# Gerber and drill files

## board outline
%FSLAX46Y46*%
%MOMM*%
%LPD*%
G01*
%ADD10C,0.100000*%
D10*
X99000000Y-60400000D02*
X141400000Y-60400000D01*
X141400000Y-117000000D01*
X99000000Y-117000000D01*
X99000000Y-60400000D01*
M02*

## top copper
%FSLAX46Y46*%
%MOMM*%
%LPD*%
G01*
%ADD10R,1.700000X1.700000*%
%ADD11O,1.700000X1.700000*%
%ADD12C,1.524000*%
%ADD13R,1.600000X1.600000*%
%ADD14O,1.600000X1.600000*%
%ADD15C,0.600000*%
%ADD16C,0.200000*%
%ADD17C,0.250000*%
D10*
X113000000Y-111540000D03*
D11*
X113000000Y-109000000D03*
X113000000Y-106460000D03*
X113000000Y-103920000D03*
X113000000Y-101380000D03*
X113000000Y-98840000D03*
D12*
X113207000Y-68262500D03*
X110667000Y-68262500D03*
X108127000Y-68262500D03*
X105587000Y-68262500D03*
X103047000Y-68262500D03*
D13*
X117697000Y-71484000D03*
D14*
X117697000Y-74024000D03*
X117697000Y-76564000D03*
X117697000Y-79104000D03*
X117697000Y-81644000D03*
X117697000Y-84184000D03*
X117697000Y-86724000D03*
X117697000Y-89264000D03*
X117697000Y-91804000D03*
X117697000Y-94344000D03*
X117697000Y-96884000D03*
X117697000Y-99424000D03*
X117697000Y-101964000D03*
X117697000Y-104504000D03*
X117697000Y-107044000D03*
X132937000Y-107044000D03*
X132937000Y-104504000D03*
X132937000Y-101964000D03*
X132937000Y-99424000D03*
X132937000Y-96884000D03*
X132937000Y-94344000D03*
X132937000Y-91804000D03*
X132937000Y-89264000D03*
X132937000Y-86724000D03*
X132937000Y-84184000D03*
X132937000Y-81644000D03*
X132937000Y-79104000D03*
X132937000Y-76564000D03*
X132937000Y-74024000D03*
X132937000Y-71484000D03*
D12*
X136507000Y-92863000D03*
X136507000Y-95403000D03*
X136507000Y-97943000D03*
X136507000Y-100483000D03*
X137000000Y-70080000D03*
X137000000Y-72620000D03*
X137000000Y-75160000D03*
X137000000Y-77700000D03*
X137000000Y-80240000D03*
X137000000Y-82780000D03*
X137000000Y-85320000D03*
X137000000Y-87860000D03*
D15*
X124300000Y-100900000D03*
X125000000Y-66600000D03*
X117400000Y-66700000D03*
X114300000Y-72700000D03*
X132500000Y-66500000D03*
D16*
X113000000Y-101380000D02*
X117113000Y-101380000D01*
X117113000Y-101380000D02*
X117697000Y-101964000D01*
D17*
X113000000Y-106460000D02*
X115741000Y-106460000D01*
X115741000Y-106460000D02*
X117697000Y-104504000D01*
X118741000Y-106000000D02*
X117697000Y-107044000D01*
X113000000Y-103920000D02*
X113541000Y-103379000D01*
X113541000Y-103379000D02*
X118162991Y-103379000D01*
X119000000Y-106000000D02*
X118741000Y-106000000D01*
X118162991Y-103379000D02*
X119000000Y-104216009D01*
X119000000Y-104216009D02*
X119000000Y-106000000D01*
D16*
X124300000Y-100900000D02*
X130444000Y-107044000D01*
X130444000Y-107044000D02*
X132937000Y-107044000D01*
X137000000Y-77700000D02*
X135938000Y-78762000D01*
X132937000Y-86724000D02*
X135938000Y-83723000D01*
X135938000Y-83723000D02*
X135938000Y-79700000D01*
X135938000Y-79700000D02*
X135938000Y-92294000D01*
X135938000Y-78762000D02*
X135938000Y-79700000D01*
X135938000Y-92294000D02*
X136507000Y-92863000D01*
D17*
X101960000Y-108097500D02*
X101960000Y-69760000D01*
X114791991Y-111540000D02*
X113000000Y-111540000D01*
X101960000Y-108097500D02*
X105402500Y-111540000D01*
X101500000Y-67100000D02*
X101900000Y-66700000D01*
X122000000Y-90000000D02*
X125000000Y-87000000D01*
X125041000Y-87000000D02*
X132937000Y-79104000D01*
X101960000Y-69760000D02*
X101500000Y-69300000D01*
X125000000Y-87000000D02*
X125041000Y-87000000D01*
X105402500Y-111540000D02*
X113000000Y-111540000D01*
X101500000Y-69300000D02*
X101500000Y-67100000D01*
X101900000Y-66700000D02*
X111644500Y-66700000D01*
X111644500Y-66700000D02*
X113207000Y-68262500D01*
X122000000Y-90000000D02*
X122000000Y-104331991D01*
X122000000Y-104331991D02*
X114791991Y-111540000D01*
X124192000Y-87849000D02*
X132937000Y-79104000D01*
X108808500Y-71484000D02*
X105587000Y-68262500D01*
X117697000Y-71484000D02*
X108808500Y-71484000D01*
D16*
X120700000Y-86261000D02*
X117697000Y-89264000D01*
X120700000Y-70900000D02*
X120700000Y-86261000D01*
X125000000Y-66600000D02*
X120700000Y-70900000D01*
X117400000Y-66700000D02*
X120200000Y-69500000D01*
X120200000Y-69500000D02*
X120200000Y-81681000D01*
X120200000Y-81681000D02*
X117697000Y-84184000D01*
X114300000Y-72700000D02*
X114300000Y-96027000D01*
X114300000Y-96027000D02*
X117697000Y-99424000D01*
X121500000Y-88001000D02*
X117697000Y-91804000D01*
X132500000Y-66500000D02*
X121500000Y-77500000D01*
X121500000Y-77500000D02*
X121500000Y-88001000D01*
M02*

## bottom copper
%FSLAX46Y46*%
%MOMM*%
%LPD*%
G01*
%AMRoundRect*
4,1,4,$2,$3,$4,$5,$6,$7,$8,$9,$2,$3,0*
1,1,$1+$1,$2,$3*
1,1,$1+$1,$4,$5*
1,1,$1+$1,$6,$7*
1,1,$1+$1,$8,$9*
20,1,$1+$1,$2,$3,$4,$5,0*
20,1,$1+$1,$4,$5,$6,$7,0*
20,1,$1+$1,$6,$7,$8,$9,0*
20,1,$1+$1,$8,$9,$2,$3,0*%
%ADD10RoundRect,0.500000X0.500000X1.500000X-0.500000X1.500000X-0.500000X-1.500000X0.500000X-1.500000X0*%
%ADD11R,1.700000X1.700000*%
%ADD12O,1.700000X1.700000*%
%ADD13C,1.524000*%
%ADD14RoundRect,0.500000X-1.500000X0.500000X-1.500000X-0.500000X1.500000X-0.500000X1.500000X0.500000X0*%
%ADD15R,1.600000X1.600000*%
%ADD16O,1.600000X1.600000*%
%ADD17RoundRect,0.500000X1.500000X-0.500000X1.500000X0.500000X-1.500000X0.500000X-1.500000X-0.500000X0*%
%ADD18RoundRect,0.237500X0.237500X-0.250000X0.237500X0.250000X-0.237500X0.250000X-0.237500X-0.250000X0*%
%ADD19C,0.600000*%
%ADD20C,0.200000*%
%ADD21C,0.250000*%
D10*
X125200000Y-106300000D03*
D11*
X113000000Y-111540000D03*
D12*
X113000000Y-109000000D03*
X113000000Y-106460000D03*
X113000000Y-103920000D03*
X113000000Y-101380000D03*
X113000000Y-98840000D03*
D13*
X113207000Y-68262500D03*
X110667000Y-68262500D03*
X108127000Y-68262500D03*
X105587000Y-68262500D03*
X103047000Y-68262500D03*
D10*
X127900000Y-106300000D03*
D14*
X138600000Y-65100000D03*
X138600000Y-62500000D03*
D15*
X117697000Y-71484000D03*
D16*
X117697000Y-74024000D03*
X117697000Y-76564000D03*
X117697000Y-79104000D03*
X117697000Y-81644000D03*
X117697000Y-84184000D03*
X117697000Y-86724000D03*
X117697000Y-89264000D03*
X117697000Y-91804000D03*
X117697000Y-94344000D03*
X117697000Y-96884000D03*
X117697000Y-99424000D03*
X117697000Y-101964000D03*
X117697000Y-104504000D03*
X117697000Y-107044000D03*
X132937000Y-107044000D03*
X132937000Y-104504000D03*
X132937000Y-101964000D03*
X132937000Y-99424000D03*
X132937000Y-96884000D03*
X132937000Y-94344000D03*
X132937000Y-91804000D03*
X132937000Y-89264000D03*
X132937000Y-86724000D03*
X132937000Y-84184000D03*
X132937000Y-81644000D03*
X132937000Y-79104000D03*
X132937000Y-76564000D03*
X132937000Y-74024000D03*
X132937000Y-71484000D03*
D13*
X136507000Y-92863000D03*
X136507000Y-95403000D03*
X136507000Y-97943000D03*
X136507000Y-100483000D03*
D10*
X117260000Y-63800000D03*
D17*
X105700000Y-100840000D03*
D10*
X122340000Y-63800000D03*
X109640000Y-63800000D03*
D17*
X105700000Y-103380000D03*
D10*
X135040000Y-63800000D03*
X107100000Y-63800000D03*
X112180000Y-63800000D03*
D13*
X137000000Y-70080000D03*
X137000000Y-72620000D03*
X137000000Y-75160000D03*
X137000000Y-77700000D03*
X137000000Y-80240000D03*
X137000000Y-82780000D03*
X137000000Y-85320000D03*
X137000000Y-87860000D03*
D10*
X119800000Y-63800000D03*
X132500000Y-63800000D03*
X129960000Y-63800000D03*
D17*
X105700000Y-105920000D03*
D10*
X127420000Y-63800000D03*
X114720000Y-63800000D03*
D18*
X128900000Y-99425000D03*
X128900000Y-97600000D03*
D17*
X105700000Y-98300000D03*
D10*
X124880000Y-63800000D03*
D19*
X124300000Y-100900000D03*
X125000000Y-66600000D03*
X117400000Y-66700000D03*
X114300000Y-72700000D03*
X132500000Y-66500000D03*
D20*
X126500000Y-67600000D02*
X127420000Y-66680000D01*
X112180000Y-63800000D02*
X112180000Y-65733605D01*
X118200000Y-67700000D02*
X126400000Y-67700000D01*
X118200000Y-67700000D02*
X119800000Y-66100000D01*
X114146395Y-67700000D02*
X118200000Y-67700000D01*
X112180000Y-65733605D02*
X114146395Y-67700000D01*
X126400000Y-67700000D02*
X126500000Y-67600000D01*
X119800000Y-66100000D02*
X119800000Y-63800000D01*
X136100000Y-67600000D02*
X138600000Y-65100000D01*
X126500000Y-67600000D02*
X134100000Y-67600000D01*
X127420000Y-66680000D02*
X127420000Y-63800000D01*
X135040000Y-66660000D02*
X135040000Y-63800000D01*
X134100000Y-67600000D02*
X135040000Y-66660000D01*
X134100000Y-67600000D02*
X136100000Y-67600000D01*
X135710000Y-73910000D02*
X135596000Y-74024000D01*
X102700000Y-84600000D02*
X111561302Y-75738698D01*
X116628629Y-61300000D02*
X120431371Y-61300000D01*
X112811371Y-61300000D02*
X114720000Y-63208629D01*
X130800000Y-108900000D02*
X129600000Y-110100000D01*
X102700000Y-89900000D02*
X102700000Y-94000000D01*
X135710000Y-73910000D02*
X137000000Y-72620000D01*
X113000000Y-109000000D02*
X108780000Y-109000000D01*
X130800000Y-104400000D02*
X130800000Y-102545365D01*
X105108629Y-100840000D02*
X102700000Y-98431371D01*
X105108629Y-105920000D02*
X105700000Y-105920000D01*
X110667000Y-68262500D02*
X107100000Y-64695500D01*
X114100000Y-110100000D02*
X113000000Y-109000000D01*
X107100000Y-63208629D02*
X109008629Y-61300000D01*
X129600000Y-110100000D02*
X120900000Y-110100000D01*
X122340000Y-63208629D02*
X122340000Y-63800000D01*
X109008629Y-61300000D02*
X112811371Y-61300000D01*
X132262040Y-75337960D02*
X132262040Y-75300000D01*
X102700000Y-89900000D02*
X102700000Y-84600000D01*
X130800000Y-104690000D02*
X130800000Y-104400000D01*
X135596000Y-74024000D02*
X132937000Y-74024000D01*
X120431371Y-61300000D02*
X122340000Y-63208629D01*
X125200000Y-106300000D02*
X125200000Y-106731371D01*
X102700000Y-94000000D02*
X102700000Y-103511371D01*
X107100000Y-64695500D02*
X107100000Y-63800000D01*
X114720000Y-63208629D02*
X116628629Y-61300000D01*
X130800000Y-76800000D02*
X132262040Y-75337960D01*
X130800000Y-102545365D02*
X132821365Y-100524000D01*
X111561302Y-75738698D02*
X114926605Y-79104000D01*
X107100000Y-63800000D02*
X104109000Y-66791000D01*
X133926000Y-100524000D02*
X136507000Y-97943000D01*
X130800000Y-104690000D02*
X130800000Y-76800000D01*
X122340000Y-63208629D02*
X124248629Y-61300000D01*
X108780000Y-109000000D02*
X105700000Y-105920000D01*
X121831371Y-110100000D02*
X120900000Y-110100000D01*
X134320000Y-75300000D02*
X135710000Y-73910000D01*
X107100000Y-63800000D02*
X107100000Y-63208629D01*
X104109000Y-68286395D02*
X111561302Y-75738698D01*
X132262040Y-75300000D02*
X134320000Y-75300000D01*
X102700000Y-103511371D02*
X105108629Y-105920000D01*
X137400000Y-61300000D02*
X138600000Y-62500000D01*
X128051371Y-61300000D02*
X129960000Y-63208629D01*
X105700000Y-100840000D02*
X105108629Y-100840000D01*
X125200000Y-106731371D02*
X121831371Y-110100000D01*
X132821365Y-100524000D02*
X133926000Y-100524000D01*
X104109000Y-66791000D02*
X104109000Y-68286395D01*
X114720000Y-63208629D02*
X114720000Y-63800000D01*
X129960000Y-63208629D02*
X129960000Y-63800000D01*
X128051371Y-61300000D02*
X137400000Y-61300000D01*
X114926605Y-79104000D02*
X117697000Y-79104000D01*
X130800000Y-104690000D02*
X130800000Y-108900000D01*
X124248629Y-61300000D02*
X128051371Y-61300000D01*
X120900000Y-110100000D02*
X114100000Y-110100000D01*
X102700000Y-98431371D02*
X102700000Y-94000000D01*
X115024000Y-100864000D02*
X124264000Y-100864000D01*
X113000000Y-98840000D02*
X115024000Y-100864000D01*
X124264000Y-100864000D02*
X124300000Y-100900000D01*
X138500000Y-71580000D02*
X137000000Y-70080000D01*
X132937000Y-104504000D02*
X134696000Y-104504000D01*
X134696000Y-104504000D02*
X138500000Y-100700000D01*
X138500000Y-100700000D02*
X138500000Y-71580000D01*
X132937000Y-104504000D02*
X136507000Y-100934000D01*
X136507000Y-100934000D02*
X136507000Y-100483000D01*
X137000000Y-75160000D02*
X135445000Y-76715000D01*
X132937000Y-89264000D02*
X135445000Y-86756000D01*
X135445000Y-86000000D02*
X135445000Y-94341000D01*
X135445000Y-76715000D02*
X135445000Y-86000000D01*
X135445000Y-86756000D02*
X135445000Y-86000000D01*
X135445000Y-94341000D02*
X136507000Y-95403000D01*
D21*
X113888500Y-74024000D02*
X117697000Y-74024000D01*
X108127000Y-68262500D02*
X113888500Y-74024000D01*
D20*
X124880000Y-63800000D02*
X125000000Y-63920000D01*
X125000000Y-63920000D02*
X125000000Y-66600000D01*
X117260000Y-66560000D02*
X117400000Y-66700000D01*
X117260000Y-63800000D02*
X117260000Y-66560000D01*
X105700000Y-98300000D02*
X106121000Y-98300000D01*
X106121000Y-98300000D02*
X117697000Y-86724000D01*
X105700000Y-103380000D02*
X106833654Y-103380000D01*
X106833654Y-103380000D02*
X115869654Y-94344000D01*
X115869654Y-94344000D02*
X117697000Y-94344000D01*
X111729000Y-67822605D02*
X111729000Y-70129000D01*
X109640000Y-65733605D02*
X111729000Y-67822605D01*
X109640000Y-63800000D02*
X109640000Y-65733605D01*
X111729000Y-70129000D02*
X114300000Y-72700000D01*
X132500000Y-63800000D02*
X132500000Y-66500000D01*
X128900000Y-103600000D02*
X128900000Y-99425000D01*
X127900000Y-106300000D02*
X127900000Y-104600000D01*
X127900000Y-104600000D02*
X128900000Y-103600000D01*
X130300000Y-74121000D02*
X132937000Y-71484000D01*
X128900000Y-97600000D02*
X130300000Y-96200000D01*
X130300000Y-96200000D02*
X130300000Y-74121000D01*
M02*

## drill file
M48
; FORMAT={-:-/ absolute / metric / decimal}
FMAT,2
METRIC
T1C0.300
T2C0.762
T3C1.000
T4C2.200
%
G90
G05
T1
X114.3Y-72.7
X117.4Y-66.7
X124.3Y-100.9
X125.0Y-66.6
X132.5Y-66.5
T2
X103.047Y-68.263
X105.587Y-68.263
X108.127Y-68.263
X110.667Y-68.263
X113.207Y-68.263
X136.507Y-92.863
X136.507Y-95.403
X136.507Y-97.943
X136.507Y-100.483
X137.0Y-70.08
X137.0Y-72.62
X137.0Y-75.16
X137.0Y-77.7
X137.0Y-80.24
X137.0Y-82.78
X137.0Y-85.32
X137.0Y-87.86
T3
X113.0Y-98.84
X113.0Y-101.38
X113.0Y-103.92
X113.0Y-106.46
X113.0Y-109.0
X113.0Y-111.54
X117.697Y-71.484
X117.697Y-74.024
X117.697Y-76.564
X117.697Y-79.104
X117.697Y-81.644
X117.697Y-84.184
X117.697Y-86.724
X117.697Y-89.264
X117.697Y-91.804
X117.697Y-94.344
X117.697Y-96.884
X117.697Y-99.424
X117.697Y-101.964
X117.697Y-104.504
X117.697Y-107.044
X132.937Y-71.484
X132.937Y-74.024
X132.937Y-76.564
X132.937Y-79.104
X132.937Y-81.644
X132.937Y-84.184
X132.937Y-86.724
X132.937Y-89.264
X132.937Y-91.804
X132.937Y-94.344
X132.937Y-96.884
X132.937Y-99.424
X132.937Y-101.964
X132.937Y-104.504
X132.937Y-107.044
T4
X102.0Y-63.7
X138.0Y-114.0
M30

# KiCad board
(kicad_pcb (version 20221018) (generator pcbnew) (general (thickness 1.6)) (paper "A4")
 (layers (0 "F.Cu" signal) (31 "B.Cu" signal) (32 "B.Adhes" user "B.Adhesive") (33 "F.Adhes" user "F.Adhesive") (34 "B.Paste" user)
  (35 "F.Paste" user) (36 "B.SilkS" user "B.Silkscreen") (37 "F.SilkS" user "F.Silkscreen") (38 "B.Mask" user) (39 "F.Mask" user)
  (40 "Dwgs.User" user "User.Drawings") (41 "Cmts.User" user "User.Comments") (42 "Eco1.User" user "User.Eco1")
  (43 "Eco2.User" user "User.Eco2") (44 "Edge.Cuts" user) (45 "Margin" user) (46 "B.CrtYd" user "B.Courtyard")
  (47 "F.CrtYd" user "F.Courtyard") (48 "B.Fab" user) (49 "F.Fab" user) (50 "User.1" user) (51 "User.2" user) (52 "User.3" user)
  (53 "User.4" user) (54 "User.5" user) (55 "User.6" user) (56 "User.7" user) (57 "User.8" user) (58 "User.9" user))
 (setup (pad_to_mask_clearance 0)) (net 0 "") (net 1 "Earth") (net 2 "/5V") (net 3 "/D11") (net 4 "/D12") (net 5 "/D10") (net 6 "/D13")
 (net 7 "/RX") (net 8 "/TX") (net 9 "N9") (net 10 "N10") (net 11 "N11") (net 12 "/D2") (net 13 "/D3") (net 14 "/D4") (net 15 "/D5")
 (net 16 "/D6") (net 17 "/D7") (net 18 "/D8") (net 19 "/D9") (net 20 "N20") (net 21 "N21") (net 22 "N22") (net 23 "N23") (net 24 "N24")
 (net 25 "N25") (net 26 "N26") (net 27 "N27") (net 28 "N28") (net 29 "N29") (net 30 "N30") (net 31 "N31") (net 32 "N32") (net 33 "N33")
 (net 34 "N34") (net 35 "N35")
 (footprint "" (layer "F.Cu") (at 125.2 106.3 90)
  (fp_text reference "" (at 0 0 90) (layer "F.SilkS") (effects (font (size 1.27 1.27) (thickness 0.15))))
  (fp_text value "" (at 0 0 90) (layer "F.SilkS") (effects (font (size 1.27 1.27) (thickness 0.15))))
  (pad "1" smd roundrect (at 0 0 180) (size 2 4) (layers "B.Cu" "B.Paste" "B.Mask") (roundrect_rratio 0.25) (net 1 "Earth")))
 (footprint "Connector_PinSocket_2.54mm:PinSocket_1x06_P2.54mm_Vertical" (layer "F.Cu") (at 113 111.54 180)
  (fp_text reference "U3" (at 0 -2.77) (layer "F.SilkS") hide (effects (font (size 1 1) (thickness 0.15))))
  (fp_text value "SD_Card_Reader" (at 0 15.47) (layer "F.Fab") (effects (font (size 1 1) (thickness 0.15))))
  (pad "1" thru_hole rect (at 0 0 180) (size 1.7 1.7) (drill 1) (layers "*.Cu" "*.Mask") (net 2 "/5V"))
  (pad "2" thru_hole oval (at 0 2.54 180) (size 1.7 1.7) (drill 1) (layers "*.Cu" "*.Mask") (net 1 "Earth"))
  (pad "3" thru_hole oval (at 0 5.08 180) (size 1.7 1.7) (drill 1) (layers "*.Cu" "*.Mask") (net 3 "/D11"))
  (pad "4" thru_hole oval (at 0 7.62 180) (size 1.7 1.7) (drill 1) (layers "*.Cu" "*.Mask") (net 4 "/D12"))
  (pad "5" thru_hole oval (at 0 10.16 180) (size 1.7 1.7) (drill 1) (layers "*.Cu" "*.Mask") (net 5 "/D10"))
  (pad "6" thru_hole oval (at 0 12.7 180) (size 1.7 1.7) (drill 1) (layers "*.Cu" "*.Mask") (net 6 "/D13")))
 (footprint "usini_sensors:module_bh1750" (layer "F.Cu") (at 103.047 68.2625 -90)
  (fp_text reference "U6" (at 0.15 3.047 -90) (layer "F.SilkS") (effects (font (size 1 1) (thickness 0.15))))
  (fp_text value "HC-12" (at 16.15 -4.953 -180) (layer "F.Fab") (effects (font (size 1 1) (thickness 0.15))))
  (pad "1" thru_hole circle (at 0 -10.16 270) (size 1.524 1.524) (drill 0.762) (layers "*.Cu" "*.Mask") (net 2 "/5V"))
  (pad "2" thru_hole circle (at 0 -7.62 270) (size 1.524 1.524) (drill 0.762) (layers "*.Cu" "*.Mask") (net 1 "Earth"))
  (pad "3" thru_hole circle (at 0 -5.08 270) (size 1.524 1.524) (drill 0.762) (layers "*.Cu" "*.Mask") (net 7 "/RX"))
  (pad "4" thru_hole circle (at 0 -2.54 270) (size 1.524 1.524) (drill 0.762) (layers "*.Cu" "*.Mask") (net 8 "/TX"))
  (pad "5" thru_hole circle (at 0 0 270) (size 1.524 1.524) (drill 0.762) (layers "*.Cu" "*.Mask") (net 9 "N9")))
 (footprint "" (layer "F.Cu") (at 127.9 106.3 90)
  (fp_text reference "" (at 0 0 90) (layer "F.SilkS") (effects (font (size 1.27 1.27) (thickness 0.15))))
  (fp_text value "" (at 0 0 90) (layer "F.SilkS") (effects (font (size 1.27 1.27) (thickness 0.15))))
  (pad "1" smd roundrect (at 0 0 180) (size 2 4) (layers "B.Cu" "B.Paste" "B.Mask") (roundrect_rratio 0.25) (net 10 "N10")))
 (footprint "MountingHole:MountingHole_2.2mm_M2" (layer "F.Cu") (at 138 114)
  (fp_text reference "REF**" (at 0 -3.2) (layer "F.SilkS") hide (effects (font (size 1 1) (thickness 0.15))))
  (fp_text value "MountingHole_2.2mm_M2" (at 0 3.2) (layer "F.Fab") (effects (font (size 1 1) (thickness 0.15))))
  (pad "" np_thru_hole circle (at 0 0) (size 2.2 2.2) (drill 2.2) (layers "*.Cu" "*.Mask")))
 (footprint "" (layer "F.Cu") (at 138.6 65.1)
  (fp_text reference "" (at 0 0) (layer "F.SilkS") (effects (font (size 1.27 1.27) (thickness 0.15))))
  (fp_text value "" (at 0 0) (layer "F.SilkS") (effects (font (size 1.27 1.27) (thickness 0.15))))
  (pad "1" smd roundrect (at 0 0 270) (size 2 4) (layers "B.Cu" "B.Paste" "B.Mask") (roundrect_rratio 0.25)))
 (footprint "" (layer "F.Cu") (at 138.6 62.5 90)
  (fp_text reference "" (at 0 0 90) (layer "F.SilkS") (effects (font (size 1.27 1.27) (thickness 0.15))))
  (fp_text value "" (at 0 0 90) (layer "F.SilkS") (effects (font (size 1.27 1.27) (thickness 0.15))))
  (pad "1" smd roundrect (at 0 0 270) (size 2 4) (layers "B.Cu" "B.Paste" "B.Mask") (roundrect_rratio 0.25) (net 1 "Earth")))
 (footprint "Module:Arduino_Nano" (layer "F.Cu") (at 117.697 71.484)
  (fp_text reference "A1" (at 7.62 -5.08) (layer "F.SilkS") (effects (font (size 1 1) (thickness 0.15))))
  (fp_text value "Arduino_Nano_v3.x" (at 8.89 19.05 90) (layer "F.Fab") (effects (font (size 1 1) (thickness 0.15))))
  (pad "1" thru_hole rect (at 0 0) (size 1.6 1.6) (drill 1) (layers "*.Cu" "*.Mask") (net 8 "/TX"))
  (pad "2" thru_hole oval (at 0 2.54) (size 1.6 1.6) (drill 1) (layers "*.Cu" "*.Mask") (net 7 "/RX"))
  (pad "3" thru_hole oval (at 0 5.08) (size 1.6 1.6) (drill 1) (layers "*.Cu" "*.Mask") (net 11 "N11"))
  (pad "4" thru_hole oval (at 0 7.62) (size 1.6 1.6) (drill 1) (layers "*.Cu" "*.Mask") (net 1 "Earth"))
  (pad "5" thru_hole oval (at 0 10.16) (size 1.6 1.6) (drill 1) (layers "*.Cu" "*.Mask") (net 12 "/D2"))
  (pad "6" thru_hole oval (at 0 12.7) (size 1.6 1.6) (drill 1) (layers "*.Cu" "*.Mask") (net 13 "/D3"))
  (pad "7" thru_hole oval (at 0 15.24) (size 1.6 1.6) (drill 1) (layers "*.Cu" "*.Mask") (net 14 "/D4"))
  (pad "8" thru_hole oval (at 0 17.78) (size 1.6 1.6) (drill 1) (layers "*.Cu" "*.Mask") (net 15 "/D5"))
  (pad "9" thru_hole oval (at 0 20.32) (size 1.6 1.6) (drill 1) (layers "*.Cu" "*.Mask") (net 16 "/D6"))
  (pad "10" thru_hole oval (at 0 22.86) (size 1.6 1.6) (drill 1) (layers "*.Cu" "*.Mask") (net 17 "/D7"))
  (pad "11" thru_hole oval (at 0 25.4) (size 1.6 1.6) (drill 1) (layers "*.Cu" "*.Mask") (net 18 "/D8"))
  (pad "12" thru_hole oval (at 0 27.94) (size 1.6 1.6) (drill 1) (layers "*.Cu" "*.Mask") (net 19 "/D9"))
  (pad "13" thru_hole oval (at 0 30.48) (size 1.6 1.6) (drill 1) (layers "*.Cu" "*.Mask") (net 5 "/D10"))
  (pad "14" thru_hole oval (at 0 33.02) (size 1.6 1.6) (drill 1) (layers "*.Cu" "*.Mask") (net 3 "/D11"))
  (pad "15" thru_hole oval (at 0 35.56) (size 1.6 1.6) (drill 1) (layers "*.Cu" "*.Mask") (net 4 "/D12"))
  (pad "16" thru_hole oval (at 15.24 35.56) (size 1.6 1.6) (drill 1) (layers "*.Cu" "*.Mask") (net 6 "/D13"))
  (pad "17" thru_hole oval (at 15.24 33.02) (size 1.6 1.6) (drill 1) (layers "*.Cu" "*.Mask") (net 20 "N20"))
  (pad "18" thru_hole oval (at 15.24 30.48) (size 1.6 1.6) (drill 1) (layers "*.Cu" "*.Mask") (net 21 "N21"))
  (pad "19" thru_hole oval (at 15.24 27.94) (size 1.6 1.6) (drill 1) (layers "*.Cu" "*.Mask") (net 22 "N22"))
  (pad "20" thru_hole oval (at 15.24 25.4) (size 1.6 1.6) (drill 1) (layers "*.Cu" "*.Mask") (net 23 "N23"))
  (pad "21" thru_hole oval (at 15.24 22.86) (size 1.6 1.6) (drill 1) (layers "*.Cu" "*.Mask") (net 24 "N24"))
  (pad "22" thru_hole oval (at 15.24 20.32) (size 1.6 1.6) (drill 1) (layers "*.Cu" "*.Mask") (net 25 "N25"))
  (pad "23" thru_hole oval (at 15.24 17.78) (size 1.6 1.6) (drill 1) (layers "*.Cu" "*.Mask") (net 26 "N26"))
  (pad "24" thru_hole oval (at 15.24 15.24) (size 1.6 1.6) (drill 1) (layers "*.Cu" "*.Mask") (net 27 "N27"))
  (pad "25" thru_hole oval (at 15.24 12.7) (size 1.6 1.6) (drill 1) (layers "*.Cu" "*.Mask") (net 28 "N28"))
  (pad "26" thru_hole oval (at 15.24 10.16) (size 1.6 1.6) (drill 1) (layers "*.Cu" "*.Mask") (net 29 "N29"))
  (pad "27" thru_hole oval (at 15.24 7.62) (size 1.6 1.6) (drill 1) (layers "*.Cu" "*.Mask") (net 2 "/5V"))
  (pad "28" thru_hole oval (at 15.24 5.08) (size 1.6 1.6) (drill 1) (layers "*.Cu" "*.Mask") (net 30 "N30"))
  (pad "29" thru_hole oval (at 15.24 2.54) (size 1.6 1.6) (drill 1) (layers "*.Cu" "*.Mask") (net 1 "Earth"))
  (pad "30" thru_hole oval (at 15.24 0) (size 1.6 1.6) (drill 1) (layers "*.Cu" "*.Mask") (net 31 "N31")))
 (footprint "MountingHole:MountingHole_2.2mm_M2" (layer "F.Cu") (at 102 63.7)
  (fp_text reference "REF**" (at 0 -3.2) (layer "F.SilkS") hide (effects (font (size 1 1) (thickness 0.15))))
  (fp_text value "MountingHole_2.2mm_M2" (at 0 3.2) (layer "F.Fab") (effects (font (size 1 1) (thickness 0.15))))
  (pad "" np_thru_hole circle (at 0 0) (size 2.2 2.2) (drill 2.2) (layers "*.Cu" "*.Mask")))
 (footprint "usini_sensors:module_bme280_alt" (layer "B.Cu") (at 136.507 100.483 180)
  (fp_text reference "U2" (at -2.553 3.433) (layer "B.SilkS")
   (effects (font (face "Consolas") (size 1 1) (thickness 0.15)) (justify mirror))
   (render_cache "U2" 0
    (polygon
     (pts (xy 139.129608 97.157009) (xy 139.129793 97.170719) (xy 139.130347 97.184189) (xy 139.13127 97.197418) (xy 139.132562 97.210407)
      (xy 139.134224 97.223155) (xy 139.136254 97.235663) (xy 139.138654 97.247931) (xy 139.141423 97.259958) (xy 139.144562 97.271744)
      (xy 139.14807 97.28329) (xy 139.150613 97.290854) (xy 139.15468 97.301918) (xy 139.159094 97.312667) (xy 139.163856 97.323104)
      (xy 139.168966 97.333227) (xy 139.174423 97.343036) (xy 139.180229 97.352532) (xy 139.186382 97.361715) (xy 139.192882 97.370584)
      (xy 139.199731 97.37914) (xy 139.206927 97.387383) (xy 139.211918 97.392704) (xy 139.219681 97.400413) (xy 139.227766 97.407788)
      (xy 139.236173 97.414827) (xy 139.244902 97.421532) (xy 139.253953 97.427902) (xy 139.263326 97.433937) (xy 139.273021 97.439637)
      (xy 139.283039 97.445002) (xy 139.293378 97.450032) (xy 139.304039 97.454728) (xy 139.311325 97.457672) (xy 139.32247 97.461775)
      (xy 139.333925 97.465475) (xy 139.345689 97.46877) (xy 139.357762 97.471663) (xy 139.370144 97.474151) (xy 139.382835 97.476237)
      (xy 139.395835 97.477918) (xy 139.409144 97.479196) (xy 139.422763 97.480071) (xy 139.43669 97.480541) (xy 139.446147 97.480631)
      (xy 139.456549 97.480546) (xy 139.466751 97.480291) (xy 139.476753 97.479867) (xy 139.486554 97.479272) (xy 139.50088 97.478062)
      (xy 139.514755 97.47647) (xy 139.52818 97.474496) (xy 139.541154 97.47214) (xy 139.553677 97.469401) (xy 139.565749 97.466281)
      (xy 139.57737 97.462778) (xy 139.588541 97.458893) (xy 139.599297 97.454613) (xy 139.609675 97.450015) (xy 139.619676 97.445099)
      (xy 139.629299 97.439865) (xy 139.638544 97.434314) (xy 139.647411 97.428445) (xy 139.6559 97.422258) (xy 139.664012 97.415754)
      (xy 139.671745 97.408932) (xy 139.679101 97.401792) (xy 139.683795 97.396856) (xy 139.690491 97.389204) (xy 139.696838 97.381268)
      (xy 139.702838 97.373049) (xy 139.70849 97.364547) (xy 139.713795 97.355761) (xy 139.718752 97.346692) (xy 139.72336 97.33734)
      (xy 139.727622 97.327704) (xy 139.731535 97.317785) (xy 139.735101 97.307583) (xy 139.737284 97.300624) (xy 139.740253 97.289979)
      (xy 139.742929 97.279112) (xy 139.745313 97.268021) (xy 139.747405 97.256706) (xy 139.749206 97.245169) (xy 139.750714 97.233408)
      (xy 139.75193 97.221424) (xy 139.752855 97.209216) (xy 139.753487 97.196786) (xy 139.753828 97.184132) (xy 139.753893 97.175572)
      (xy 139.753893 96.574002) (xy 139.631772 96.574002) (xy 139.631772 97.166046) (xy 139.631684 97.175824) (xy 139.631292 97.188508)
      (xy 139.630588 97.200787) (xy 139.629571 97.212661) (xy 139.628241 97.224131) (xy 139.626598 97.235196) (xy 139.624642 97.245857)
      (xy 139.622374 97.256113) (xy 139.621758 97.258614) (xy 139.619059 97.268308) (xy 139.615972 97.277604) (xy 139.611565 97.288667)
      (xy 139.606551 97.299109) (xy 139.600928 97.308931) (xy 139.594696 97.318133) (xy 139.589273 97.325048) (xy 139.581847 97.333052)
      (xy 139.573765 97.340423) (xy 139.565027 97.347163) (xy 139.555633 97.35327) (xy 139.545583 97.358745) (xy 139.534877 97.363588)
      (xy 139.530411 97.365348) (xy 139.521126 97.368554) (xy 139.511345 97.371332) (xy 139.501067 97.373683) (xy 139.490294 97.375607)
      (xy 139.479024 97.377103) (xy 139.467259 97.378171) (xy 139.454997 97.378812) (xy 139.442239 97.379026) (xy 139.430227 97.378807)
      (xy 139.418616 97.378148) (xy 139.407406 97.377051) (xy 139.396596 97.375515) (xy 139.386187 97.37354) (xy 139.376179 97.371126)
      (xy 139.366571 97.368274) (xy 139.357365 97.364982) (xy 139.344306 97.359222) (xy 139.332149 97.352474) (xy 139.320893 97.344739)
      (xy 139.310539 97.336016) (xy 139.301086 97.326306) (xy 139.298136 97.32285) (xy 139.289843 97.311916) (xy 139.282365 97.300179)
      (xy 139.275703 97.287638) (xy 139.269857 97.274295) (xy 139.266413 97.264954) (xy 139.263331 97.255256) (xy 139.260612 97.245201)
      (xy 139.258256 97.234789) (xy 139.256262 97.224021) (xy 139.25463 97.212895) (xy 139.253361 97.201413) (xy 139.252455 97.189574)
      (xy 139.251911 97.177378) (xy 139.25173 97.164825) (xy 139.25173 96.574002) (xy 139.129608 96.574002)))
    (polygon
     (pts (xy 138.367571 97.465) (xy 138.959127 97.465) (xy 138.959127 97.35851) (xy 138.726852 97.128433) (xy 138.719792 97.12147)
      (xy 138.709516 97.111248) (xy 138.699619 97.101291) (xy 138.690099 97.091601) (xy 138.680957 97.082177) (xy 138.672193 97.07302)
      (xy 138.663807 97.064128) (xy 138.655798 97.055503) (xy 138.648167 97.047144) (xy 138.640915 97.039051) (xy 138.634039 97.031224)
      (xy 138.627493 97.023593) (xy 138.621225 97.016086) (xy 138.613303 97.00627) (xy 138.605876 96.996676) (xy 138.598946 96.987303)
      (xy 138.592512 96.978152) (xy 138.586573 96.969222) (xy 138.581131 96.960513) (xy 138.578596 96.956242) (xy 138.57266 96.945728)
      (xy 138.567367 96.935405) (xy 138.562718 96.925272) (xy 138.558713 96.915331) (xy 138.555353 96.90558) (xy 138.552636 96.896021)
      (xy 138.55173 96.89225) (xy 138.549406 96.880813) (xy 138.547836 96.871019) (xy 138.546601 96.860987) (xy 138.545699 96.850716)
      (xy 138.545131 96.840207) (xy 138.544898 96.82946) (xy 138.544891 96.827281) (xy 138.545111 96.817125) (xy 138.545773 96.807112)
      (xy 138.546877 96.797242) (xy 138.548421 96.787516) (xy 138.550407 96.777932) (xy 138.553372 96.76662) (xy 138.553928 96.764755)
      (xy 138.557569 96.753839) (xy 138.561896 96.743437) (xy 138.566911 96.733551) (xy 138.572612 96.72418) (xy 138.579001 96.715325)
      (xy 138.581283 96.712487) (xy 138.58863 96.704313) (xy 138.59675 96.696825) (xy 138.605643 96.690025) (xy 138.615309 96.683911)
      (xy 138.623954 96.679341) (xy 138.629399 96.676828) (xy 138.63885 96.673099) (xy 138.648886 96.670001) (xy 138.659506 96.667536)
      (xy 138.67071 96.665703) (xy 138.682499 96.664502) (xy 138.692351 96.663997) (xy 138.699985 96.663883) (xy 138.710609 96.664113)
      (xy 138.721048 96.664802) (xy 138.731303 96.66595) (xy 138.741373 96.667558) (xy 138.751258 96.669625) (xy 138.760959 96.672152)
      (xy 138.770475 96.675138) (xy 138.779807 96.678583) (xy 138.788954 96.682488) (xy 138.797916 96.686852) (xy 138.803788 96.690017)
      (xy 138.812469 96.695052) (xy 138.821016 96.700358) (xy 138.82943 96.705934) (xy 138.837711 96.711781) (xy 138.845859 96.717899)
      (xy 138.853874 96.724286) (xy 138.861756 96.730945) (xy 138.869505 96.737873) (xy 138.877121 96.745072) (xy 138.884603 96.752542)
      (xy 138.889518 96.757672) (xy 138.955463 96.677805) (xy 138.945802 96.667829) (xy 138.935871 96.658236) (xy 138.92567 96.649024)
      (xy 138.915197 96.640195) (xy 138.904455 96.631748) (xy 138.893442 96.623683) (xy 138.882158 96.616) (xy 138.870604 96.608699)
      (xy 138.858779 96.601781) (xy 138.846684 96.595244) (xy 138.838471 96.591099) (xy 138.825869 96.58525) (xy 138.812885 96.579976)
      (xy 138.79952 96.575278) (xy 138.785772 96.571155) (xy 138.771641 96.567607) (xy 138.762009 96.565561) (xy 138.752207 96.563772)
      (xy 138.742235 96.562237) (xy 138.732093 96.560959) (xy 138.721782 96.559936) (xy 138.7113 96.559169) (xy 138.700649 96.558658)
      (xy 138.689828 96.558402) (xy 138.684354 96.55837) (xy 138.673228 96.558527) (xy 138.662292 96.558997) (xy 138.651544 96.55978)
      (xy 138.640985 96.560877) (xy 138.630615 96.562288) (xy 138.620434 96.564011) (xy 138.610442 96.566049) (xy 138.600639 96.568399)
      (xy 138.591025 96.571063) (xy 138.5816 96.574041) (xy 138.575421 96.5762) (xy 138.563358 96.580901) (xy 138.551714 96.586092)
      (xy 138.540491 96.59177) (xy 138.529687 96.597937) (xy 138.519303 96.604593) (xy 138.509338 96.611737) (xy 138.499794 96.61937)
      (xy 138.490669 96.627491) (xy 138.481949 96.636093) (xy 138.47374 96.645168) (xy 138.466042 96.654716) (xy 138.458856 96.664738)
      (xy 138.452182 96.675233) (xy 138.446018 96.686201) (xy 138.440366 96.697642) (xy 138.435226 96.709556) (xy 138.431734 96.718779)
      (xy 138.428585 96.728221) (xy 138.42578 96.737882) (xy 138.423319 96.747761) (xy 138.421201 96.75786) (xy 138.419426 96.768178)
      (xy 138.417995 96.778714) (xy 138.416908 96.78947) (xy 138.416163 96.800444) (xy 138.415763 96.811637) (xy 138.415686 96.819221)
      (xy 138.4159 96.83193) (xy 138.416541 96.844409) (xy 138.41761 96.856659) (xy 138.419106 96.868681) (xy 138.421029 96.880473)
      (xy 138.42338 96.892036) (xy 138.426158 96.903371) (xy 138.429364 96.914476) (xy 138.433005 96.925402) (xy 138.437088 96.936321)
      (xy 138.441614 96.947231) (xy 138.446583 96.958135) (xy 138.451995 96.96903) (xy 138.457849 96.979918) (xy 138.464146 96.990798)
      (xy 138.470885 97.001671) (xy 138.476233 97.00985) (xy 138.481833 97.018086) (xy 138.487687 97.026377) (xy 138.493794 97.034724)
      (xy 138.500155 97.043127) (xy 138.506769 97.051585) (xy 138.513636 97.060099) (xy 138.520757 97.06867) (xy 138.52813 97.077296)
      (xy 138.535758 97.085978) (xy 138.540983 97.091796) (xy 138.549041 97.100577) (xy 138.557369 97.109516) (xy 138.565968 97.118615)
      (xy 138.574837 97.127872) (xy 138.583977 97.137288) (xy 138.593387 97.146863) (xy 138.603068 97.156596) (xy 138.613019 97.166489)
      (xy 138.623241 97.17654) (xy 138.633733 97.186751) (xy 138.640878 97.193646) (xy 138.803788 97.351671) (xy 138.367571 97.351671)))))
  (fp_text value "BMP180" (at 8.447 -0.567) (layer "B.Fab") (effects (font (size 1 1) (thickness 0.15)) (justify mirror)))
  (pad "1" thru_hole circle (at 0 7.62 180) (size 1.524 1.524) (drill 0.762) (layers "*.Cu" "*.Mask") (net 27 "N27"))
  (pad "2" thru_hole circle (at 0 5.08 180) (size 1.524 1.524) (drill 0.762) (layers "*.Cu" "*.Mask") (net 26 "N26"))
  (pad "3" thru_hole circle (at 0 2.54 180) (size 1.524 1.524) (drill 0.762) (layers "*.Cu" "*.Mask") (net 1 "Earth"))
  (pad "4" thru_hole circle (at 0 0 180) (size 1.524 1.524) (drill 0.762) (layers "*.Cu" "*.Mask") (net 20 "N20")))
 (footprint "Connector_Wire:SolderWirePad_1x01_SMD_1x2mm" (layer "B.Cu") (at 117.26 63.8 180)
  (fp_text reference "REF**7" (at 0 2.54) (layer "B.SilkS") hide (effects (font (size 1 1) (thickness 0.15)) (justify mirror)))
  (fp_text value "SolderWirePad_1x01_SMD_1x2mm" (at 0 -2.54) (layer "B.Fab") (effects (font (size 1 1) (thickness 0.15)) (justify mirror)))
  (pad "1" smd roundrect (at 0 0 180) (size 2 4) (layers "B.Cu" "B.Paste" "B.Mask") (roundrect_rratio 0.25) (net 13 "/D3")))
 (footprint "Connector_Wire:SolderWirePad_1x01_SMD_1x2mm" (layer "B.Cu") (at 105.7 100.84 90)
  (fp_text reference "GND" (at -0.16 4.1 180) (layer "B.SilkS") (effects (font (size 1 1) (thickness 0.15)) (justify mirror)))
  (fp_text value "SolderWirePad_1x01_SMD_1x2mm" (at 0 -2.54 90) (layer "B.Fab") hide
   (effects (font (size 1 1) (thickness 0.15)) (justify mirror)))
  (pad "1" smd roundrect (at 0 0 90) (size 2 4) (layers "B.Cu" "B.Paste" "B.Mask") (roundrect_rratio 0.25) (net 1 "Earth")))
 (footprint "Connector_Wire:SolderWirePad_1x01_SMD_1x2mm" (layer "B.Cu") (at 122.34 63.8 180)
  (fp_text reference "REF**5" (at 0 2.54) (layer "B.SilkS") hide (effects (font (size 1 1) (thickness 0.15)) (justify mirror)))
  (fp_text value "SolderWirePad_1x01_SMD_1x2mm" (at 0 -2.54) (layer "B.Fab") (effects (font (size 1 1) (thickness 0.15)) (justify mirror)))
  (pad "1" smd roundrect (at 0 0 180) (size 2 4) (layers "B.Cu" "B.Paste" "B.Mask") (roundrect_rratio 0.25) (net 1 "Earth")))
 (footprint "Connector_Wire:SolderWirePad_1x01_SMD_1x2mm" (layer "B.Cu") (at 109.64 63.8 180)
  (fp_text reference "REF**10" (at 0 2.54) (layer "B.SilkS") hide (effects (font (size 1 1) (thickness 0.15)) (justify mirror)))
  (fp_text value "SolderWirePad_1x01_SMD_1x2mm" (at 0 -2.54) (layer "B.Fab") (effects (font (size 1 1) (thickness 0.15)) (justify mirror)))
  (pad "1" smd roundrect (at 0 0 180) (size 2 4) (layers "B.Cu" "B.Paste" "B.Mask") (roundrect_rratio 0.25) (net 19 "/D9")))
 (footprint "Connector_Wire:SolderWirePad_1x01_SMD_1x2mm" (layer "B.Cu") (at 105.7 103.38 90)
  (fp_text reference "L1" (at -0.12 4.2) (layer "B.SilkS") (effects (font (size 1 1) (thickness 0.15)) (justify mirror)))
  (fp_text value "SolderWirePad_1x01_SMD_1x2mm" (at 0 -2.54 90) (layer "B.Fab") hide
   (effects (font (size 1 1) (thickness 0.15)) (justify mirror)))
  (pad "1" smd roundrect (at 0 0 90) (size 2 4) (layers "B.Cu" "B.Paste" "B.Mask") (roundrect_rratio 0.25) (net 17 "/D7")))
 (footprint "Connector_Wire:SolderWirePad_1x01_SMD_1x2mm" (layer "B.Cu") (at 135.04 63.8 180)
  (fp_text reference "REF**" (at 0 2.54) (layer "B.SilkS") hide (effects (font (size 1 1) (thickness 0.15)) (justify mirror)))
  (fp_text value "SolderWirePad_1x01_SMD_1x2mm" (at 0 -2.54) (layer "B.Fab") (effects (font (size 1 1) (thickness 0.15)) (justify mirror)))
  (pad "1" smd roundrect (at 0 0 180) (size 2 4) (layers "B.Cu" "B.Paste" "B.Mask") (roundrect_rratio 0.25)))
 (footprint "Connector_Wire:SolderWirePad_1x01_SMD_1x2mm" (layer "B.Cu") (at 107.1 63.8 180)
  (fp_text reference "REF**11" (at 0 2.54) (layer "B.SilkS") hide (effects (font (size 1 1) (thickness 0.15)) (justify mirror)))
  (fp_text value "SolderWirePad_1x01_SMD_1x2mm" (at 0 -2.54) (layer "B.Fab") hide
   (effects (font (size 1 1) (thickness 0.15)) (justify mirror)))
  (pad "1" smd roundrect (at 0 0 180) (size 2 4) (layers "B.Cu" "B.Paste" "B.Mask") (roundrect_rratio 0.25) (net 1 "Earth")))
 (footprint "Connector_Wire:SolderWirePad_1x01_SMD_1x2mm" (layer "B.Cu") (at 112.18 63.8 180)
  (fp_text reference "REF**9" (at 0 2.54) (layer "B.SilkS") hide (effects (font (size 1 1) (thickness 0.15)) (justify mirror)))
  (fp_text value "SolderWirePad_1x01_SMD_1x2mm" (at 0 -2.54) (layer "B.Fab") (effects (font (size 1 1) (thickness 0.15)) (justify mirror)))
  (pad "1" smd roundrect (at 0 0 180) (size 2 4) (layers "B.Cu" "B.Paste" "B.Mask") (roundrect_rratio 0.25)))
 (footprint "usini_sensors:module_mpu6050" (layer "B.Cu") (at 137 87.86 180)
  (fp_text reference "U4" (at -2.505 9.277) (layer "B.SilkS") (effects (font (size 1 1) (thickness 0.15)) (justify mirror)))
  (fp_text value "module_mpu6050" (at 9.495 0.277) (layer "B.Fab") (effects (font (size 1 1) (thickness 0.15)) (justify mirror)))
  (pad "1" thru_hole circle (at 0 17.78 180) (size 1.524 1.524) (drill 0.762) (layers "*.Cu" "*.Mask") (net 20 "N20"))
  (pad "2" thru_hole circle (at 0 15.24 180) (size 1.524 1.524) (drill 0.762) (layers "*.Cu" "*.Mask") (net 1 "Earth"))
  (pad "3" thru_hole circle (at 0 12.7 180) (size 1.524 1.524) (drill 0.762) (layers "*.Cu" "*.Mask") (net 26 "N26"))
  (pad "4" thru_hole circle (at 0 10.16 180) (size 1.524 1.524) (drill 0.762) (layers "*.Cu" "*.Mask") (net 27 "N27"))
  (pad "5" thru_hole circle (at 0 7.62 180) (size 1.524 1.524) (drill 0.762) (layers "*.Cu" "*.Mask") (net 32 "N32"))
  (pad "6" thru_hole circle (at 0 5.08 180) (size 1.524 1.524) (drill 0.762) (layers "*.Cu" "*.Mask") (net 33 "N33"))
  (pad "7" thru_hole circle (at 0 2.54 180) (size 1.524 1.524) (drill 0.762) (layers "*.Cu" "*.Mask") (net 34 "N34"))
  (pad "8" thru_hole circle (at 0 0 180) (size 1.524 1.524) (drill 0.762) (layers "*.Cu" "*.Mask") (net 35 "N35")))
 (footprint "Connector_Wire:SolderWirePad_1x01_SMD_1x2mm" (layer "B.Cu") (at 119.8 63.8 180)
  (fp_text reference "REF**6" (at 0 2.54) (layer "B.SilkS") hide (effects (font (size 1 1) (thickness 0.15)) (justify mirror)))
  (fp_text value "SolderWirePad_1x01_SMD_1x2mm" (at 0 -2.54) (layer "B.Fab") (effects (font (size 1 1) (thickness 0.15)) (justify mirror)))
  (pad "1" smd roundrect (at 0 0 180) (size 2 4) (layers "B.Cu" "B.Paste" "B.Mask") (roundrect_rratio 0.25)))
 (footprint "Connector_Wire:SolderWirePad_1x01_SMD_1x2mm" (layer "B.Cu") (at 132.5 63.8 180)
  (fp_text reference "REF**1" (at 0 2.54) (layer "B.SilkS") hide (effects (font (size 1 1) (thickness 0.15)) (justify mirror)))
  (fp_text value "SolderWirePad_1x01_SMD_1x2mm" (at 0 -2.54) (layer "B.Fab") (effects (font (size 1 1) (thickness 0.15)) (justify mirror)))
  (pad "1" smd roundrect (at 0 0 180) (size 2 4) (layers "B.Cu" "B.Paste" "B.Mask") (roundrect_rratio 0.25) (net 16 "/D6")))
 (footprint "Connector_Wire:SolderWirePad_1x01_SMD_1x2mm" (layer "B.Cu") (at 129.96 63.8 180)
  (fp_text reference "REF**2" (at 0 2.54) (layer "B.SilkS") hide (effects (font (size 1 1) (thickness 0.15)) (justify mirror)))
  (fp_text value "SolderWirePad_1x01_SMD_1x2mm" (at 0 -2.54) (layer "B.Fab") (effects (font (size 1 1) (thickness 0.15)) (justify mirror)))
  (pad "1" smd roundrect (at 0 0 180) (size 2 4) (layers "B.Cu" "B.Paste" "B.Mask") (roundrect_rratio 0.25) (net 1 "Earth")))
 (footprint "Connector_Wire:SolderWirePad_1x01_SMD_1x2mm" (layer "B.Cu") (at 105.7 105.92 90)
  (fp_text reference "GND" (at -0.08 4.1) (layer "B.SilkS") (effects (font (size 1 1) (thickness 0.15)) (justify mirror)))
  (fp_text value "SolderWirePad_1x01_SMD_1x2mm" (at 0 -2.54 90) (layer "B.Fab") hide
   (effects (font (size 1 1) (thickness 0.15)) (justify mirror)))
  (pad "1" smd roundrect (at 0 0 90) (size 2 4) (layers "B.Cu" "B.Paste" "B.Mask") (roundrect_rratio 0.25) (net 1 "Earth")))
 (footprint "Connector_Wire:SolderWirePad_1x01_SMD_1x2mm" (layer "B.Cu") (at 127.42 63.8 180)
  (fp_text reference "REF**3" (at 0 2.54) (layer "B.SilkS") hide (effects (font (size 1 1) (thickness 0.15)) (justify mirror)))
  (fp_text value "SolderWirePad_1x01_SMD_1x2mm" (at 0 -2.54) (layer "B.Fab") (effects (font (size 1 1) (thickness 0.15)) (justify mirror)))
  (pad "1" smd roundrect (at 0 0 180) (size 2 4) (layers "B.Cu" "B.Paste" "B.Mask") (roundrect_rratio 0.25)))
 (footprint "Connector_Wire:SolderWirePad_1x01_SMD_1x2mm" (layer "B.Cu") (at 114.72 63.8 180)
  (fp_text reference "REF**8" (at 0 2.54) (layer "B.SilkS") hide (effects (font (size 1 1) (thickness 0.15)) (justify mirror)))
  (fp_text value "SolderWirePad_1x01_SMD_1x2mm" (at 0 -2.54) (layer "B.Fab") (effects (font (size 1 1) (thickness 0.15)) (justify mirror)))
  (pad "1" smd roundrect (at 0 0 180) (size 2 4) (layers "B.Cu" "B.Paste" "B.Mask") (roundrect_rratio 0.25) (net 1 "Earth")))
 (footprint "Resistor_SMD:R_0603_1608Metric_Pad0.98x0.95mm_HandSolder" (layer "B.Cu") (at 128.9 98.5125 90)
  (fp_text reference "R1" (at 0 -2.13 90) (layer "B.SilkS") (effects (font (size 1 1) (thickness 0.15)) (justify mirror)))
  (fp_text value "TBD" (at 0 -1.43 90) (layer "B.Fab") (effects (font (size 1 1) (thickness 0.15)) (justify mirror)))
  (pad "1" smd roundrect (at -0.9125 0 90) (size 0.975 0.95) (layers "B.Cu" "B.Paste" "B.Mask") (roundrect_rratio 0.25) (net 10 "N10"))
  (pad "2" smd roundrect (at 0.9125 0 90) (size 0.975 0.95) (layers "B.Cu" "B.Paste" "B.Mask") (roundrect_rratio 0.25) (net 31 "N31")))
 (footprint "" (layer "B.Cu") (at 105.7 98.3 90)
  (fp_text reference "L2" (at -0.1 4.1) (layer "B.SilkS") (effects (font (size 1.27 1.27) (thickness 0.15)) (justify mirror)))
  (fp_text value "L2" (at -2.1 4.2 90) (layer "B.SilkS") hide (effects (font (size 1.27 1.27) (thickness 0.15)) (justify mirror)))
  (pad "1" smd roundrect (at 0 0 90) (size 2 4) (layers "B.Cu" "B.Paste" "B.Mask") (roundrect_rratio 0.25) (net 14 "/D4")))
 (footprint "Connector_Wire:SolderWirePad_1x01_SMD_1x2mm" (layer "B.Cu") (at 124.88 63.8 180)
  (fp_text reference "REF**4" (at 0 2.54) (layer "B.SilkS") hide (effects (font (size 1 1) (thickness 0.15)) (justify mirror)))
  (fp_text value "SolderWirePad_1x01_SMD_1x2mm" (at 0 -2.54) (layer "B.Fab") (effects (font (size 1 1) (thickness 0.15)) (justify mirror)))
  (pad "1" smd roundrect (at 0 0 180) (size 2 4) (layers "B.Cu" "B.Paste" "B.Mask") (roundrect_rratio 0.25) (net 15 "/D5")))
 (gr_rect (start 99 60.4) (end 141.4 117) (stroke (width 0.1) (type default)) (fill none) (layer "Edge.Cuts"))
 (segment (start 126.5 67.6) (end 127.42 66.68) (width 0.2) (layer "B.Cu") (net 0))
 (segment (start 112.18 63.8) (end 112.18 65.733605) (width 0.2) (layer "B.Cu") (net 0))
 (segment (start 118.2 67.7) (end 126.4 67.7) (width 0.2) (layer "B.Cu") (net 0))
 (segment (start 118.2 67.7) (end 119.8 66.1) (width 0.2) (layer "B.Cu") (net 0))
 (segment (start 114.146395 67.7) (end 118.2 67.7) (width 0.2) (layer "B.Cu") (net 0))
 (segment (start 112.18 65.733605) (end 114.146395 67.7) (width 0.2) (layer "B.Cu") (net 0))
 (segment (start 126.4 67.7) (end 126.5 67.6) (width 0.2) (layer "B.Cu") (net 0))
 (segment (start 119.8 66.1) (end 119.8 63.8) (width 0.2) (layer "B.Cu") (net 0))
 (segment (start 136.1 67.6) (end 138.6 65.1) (width 0.2) (layer "B.Cu") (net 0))
 (segment (start 126.5 67.6) (end 134.1 67.6) (width 0.2) (layer "B.Cu") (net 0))
 (segment (start 127.42 66.68) (end 127.42 63.8) (width 0.2) (layer "B.Cu") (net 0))
 (segment (start 135.04 66.66) (end 135.04 63.8) (width 0.2) (layer "B.Cu") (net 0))
 (segment (start 134.1 67.6) (end 135.04 66.66) (width 0.2) (layer "B.Cu") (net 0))
 (segment (start 134.1 67.6) (end 136.1 67.6) (width 0.2) (layer "B.Cu") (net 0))
 (segment (start 135.71 73.91) (end 135.596 74.024) (width 0.2) (layer "B.Cu") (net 1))
 (segment (start 102.7 84.6) (end 111.561302 75.738698) (width 0.2) (layer "B.Cu") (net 1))
 (segment (start 116.628629 61.3) (end 120.431371 61.3) (width 0.2) (layer "B.Cu") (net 1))
 (segment (start 112.811371 61.3) (end 114.72 63.208629) (width 0.2) (layer "B.Cu") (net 1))
 (segment (start 130.8 108.9) (end 129.6 110.1) (width 0.2) (layer "B.Cu") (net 1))
 (segment (start 102.7 89.9) (end 102.7 94) (width 0.2) (layer "B.Cu") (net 1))
 (segment (start 135.71 73.91) (end 137 72.62) (width 0.2) (layer "B.Cu") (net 1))
 (segment (start 113 109) (end 108.78 109) (width 0.2) (layer "B.Cu") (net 1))
 (segment (start 130.8 104.4) (end 130.8 102.545365) (width 0.2) (layer "B.Cu") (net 1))
 (segment (start 105.108629 100.84) (end 102.7 98.431371) (width 0.2) (layer "B.Cu") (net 1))
 (segment (start 105.108629 105.92) (end 105.7 105.92) (width 0.2) (layer "B.Cu") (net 1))
 (segment (start 110.667 68.2625) (end 107.1 64.6955) (width 0.2) (layer "B.Cu") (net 1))
 (segment (start 114.1 110.1) (end 113 109) (width 0.2) (layer "B.Cu") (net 1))
 (segment (start 107.1 63.208629) (end 109.008629 61.3) (width 0.2) (layer "B.Cu") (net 1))
 (segment (start 129.6 110.1) (end 120.9 110.1) (width 0.2) (layer "B.Cu") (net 1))
 (segment (start 122.34 63.208629) (end 122.34 63.8) (width 0.2) (layer "B.Cu") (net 1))
 (segment (start 109.008629 61.3) (end 112.811371 61.3) (width 0.2) (layer "B.Cu") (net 1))
 (segment (start 132.26204 75.33796) (end 132.26204 75.3) (width 0.2) (layer "B.Cu") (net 1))
 (segment (start 102.7 89.9) (end 102.7 84.6) (width 0.2) (layer "B.Cu") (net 1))
 (segment (start 130.8 104.69) (end 130.8 104.4) (width 0.2) (layer "B.Cu") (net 1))
 (segment (start 135.596 74.024) (end 132.937 74.024) (width 0.2) (layer "B.Cu") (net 1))
 (segment (start 120.431371 61.3) (end 122.34 63.208629) (width 0.2) (layer "B.Cu") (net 1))
 (segment (start 125.2 106.3) (end 125.2 106.731371) (width 0.2) (layer "B.Cu") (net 1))
 (segment (start 102.7 94) (end 102.7 103.511371) (width 0.2) (layer "B.Cu") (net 1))
 (segment (start 107.1 64.6955) (end 107.1 63.8) (width 0.2) (layer "B.Cu") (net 1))
 (segment (start 114.72 63.208629) (end 116.628629 61.3) (width 0.2) (layer "B.Cu") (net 1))
 (segment (start 130.8 76.8) (end 132.26204 75.33796) (width 0.2) (layer "B.Cu") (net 1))
 (segment (start 130.8 102.545365) (end 132.821365 100.524) (width 0.2) (layer "B.Cu") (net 1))
 (segment (start 111.561302 75.738698) (end 114.926605 79.104) (width 0.2) (layer "B.Cu") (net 1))
 (segment (start 107.1 63.8) (end 104.109 66.791) (width 0.2) (layer "B.Cu") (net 1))
 (segment (start 133.926 100.524) (end 136.507 97.943) (width 0.2) (layer "B.Cu") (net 1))
 (segment (start 130.8 104.69) (end 130.8 76.8) (width 0.2) (layer "B.Cu") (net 1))
 (segment (start 122.34 63.208629) (end 124.248629 61.3) (width 0.2) (layer "B.Cu") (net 1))
 (segment (start 108.78 109) (end 105.7 105.92) (width 0.2) (layer "B.Cu") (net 1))
 (segment (start 121.831371 110.1) (end 120.9 110.1) (width 0.2) (layer "B.Cu") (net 1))
 (segment (start 134.32 75.3) (end 135.71 73.91) (width 0.2) (layer "B.Cu") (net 1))
 (segment (start 107.1 63.8) (end 107.1 63.208629) (width 0.2) (layer "B.Cu") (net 1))
 (segment (start 104.109 68.286395) (end 111.561302 75.738698) (width 0.2) (layer "B.Cu") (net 1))
 (segment (start 132.26204 75.3) (end 134.32 75.3) (width 0.2) (layer "B.Cu") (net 1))
 (segment (start 102.7 103.511371) (end 105.108629 105.92) (width 0.2) (layer "B.Cu") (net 1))
 (segment (start 137.4 61.3) (end 138.6 62.5) (width 0.2) (layer "B.Cu") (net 1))
 (segment (start 128.051371 61.3) (end 129.96 63.208629) (width 0.2) (layer "B.Cu") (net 1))
 (segment (start 105.7 100.84) (end 105.108629 100.84) (width 0.2) (layer "B.Cu") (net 1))
 (segment (start 125.2 106.731371) (end 121.831371 110.1) (width 0.2) (layer "B.Cu") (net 1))
 (segment (start 132.821365 100.524) (end 133.926 100.524) (width 0.2) (layer "B.Cu") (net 1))
 (segment (start 104.109 66.791) (end 104.109 68.286395) (width 0.2) (layer "B.Cu") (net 1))
 (segment (start 114.72 63.208629) (end 114.72 63.8) (width 0.2) (layer "B.Cu") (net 1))
 (segment (start 129.96 63.208629) (end 129.96 63.8) (width 0.2) (layer "B.Cu") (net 1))
 (segment (start 128.051371 61.3) (end 137.4 61.3) (width 0.2) (layer "B.Cu") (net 1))
 (segment (start 114.926605 79.104) (end 117.697 79.104) (width 0.2) (layer "B.Cu") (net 1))
 (segment (start 130.8 104.69) (end 130.8 108.9) (width 0.2) (layer "B.Cu") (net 1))
 (segment (start 124.248629 61.3) (end 128.051371 61.3) (width 0.2) (layer "B.Cu") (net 1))
 (segment (start 120.9 110.1) (end 114.1 110.1) (width 0.2) (layer "B.Cu") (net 1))
 (segment (start 102.7 98.431371) (end 102.7 94) (width 0.2) (layer "B.Cu") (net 1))
 (segment (start 113 101.38) (end 117.113 101.38) (width 0.2) (layer "F.Cu") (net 5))
 (segment (start 117.113 101.38) (end 117.697 101.964) (width 0.2) (layer "F.Cu") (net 5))
 (segment (start 113 106.46) (end 115.741 106.46) (width 0.25) (layer "F.Cu") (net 3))
 (segment (start 115.741 106.46) (end 117.697 104.504) (width 0.25) (layer "F.Cu") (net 3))
 (segment (start 118.741 106) (end 117.697 107.044) (width 0.25) (layer "F.Cu") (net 4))
 (segment (start 113 103.92) (end 113.541 103.379) (width 0.25) (layer "F.Cu") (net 4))
 (segment (start 113.541 103.379) (end 118.162991 103.379) (width 0.25) (layer "F.Cu") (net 4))
 (segment (start 119 106) (end 118.741 106) (width 0.25) (layer "F.Cu") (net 4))
 (segment (start 118.162991 103.379) (end 119 104.216009) (width 0.25) (layer "F.Cu") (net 4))
 (segment (start 119 104.216009) (end 119 106) (width 0.25) (layer "F.Cu") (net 4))
 (segment (start 124.3 100.9) (end 130.444 107.044) (width 0.2) (layer "F.Cu") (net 6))
 (segment (start 130.444 107.044) (end 132.937 107.044) (width 0.2) (layer "F.Cu") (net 6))
 (via (at 124.3 100.9) (size 0.6) (drill 0.3) (layers "F.Cu" "B.Cu") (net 6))
 (segment (start 115.024 100.864) (end 124.264 100.864) (width 0.2) (layer "B.Cu") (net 6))
 (segment (start 113 98.84) (end 115.024 100.864) (width 0.2) (layer "B.Cu") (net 6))
 (segment (start 124.264 100.864) (end 124.3 100.9) (width 0.2) (layer "B.Cu") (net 6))
 (segment (start 138.5 71.58) (end 137 70.08) (width 0.2) (layer "B.Cu") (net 20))
 (segment (start 132.937 104.504) (end 134.696 104.504) (width 0.2) (layer "B.Cu") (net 20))
 (segment (start 134.696 104.504) (end 138.5 100.7) (width 0.2) (layer "B.Cu") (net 20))
 (segment (start 138.5 100.7) (end 138.5 71.58) (width 0.2) (layer "B.Cu") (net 20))
 (segment (start 132.937 104.504) (end 136.507 100.934) (width 0.2) (layer "B.Cu") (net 20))
 (segment (start 136.507 100.934) (end 136.507 100.483) (width 0.2) (layer "B.Cu") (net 20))
 (segment (start 137 75.16) (end 135.445 76.715) (width 0.2) (layer "B.Cu") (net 26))
 (segment (start 132.937 89.264) (end 135.445 86.756) (width 0.2) (layer "B.Cu") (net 26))
 (segment (start 135.445 86) (end 135.445 94.341) (width 0.2) (layer "B.Cu") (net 26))
 (segment (start 135.445 76.715) (end 135.445 86) (width 0.2) (layer "B.Cu") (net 26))
 (segment (start 135.445 86.756) (end 135.445 86) (width 0.2) (layer "B.Cu") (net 26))
 (segment (start 135.445 94.341) (end 136.507 95.403) (width 0.2) (layer "B.Cu") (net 26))
 (segment (start 137 77.7) (end 135.938 78.762) (width 0.2) (layer "F.Cu") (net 27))
 (segment (start 132.937 86.724) (end 135.938 83.723) (width 0.2) (layer "F.Cu") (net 27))
 (segment (start 135.938 83.723) (end 135.938 79.7) (width 0.2) (layer "F.Cu") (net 27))
 (segment (start 135.938 79.7) (end 135.938 92.294) (width 0.2) (layer "F.Cu") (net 27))
 (segment (start 135.938 78.762) (end 135.938 79.7) (width 0.2) (layer "F.Cu") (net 27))
 (segment (start 135.938 92.294) (end 136.507 92.863) (width 0.2) (layer "F.Cu") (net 27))
 (segment (start 101.96 108.0975) (end 101.96 69.76) (width 0.25) (layer "F.Cu") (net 2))
 (segment (start 114.791991 111.54) (end 113 111.54) (width 0.25) (layer "F.Cu") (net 2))
 (segment (start 101.96 108.0975) (end 105.4025 111.54) (width 0.25) (layer "F.Cu") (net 2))
 (segment (start 101.5 67.1) (end 101.9 66.7) (width 0.25) (layer "F.Cu") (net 2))
 (segment (start 122 90) (end 125 87) (width 0.25) (layer "F.Cu") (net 2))
 (segment (start 125.041 87) (end 132.937 79.104) (width 0.25) (layer "F.Cu") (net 2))
 (segment (start 101.96 69.76) (end 101.5 69.3) (width 0.25) (layer "F.Cu") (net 2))
 (segment (start 125 87) (end 125.041 87) (width 0.25) (layer "F.Cu") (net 2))
 (segment (start 105.4025 111.54) (end 113 111.54) (width 0.25) (layer "F.Cu") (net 2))
 (segment (start 101.5 69.3) (end 101.5 67.1) (width 0.25) (layer "F.Cu") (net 2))
 (segment (start 101.9 66.7) (end 111.6445 66.7) (width 0.25) (layer "F.Cu") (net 2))
 (segment (start 111.6445 66.7) (end 113.207 68.2625) (width 0.25) (layer "F.Cu") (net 2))
 (segment (start 122 90) (end 122 104.331991) (width 0.25) (layer "F.Cu") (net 2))
 (segment (start 122 104.331991) (end 114.791991 111.54) (width 0.25) (layer "F.Cu") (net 2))
 (segment (start 124.192 87.849) (end 132.937 79.104) (width 0.25) (layer "F.Cu") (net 2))
 (segment (start 108.8085 71.484) (end 105.587 68.2625) (width 0.25) (layer "F.Cu") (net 8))
 (segment (start 117.697 71.484) (end 108.8085 71.484) (width 0.25) (layer "F.Cu") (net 8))
 (segment (start 113.8885 74.024) (end 117.697 74.024) (width 0.25) (layer "B.Cu") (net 7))
 (segment (start 108.127 68.2625) (end 113.8885 74.024) (width 0.25) (layer "B.Cu") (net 7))
 (segment (start 120.7 86.261) (end 117.697 89.264) (width 0.2) (layer "F.Cu") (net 15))
 (segment (start 120.7 70.9) (end 120.7 86.261) (width 0.2) (layer "F.Cu") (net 15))
 (segment (start 125 66.6) (end 120.7 70.9) (width 0.2) (layer "F.Cu") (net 15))
 (via (at 125 66.6) (size 0.6) (drill 0.3) (layers "F.Cu" "B.Cu") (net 15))
 (segment (start 124.88 63.8) (end 125 63.92) (width 0.2) (layer "B.Cu") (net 15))
 (segment (start 125 63.92) (end 125 66.6) (width 0.2) (layer "B.Cu") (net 15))
 (segment (start 117.4 66.7) (end 120.2 69.5) (width 0.2) (layer "F.Cu") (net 13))
 (segment (start 120.2 69.5) (end 120.2 81.681) (width 0.2) (layer "F.Cu") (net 13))
 (segment (start 120.2 81.681) (end 117.697 84.184) (width 0.2) (layer "F.Cu") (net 13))
 (via (at 117.4 66.7) (size 0.6) (drill 0.3) (layers "F.Cu" "B.Cu") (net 13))
 (segment (start 117.26 66.56) (end 117.4 66.7) (width 0.2) (layer "B.Cu") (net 13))
 (segment (start 117.26 63.8) (end 117.26 66.56) (width 0.2) (layer "B.Cu") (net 13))
 (segment (start 105.7 98.3) (end 106.121 98.3) (width 0.2) (layer "B.Cu") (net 14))
 (segment (start 106.121 98.3) (end 117.697 86.724) (width 0.2) (layer "B.Cu") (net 14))
 (segment (start 105.7 103.38) (end 106.833654 103.38) (width 0.2) (layer "B.Cu") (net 17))
 (segment (start 106.833654 103.38) (end 115.869654 94.344) (width 0.2) (layer "B.Cu") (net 17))
 (segment (start 115.869654 94.344) (end 117.697 94.344) (width 0.2) (layer "B.Cu") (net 17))
 (segment (start 114.3 72.7) (end 114.3 96.027) (width 0.2) (layer "F.Cu") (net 19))
 (segment (start 114.3 96.027) (end 117.697 99.424) (width 0.2) (layer "F.Cu") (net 19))
 (via (at 114.3 72.7) (size 0.6) (drill 0.3) (layers "F.Cu" "B.Cu") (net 19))
 (segment (start 111.729 67.822605) (end 111.729 70.129) (width 0.2) (layer "B.Cu") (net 19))
 (segment (start 109.64 65.733605) (end 111.729 67.822605) (width 0.2) (layer "B.Cu") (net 19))
 (segment (start 109.64 63.8) (end 109.64 65.733605) (width 0.2) (layer "B.Cu") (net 19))
 (segment (start 111.729 70.129) (end 114.3 72.7) (width 0.2) (layer "B.Cu") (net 19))
 (segment (start 121.5 88.001) (end 117.697 91.804) (width 0.2) (layer "F.Cu") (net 16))
 (segment (start 132.5 66.5) (end 121.5 77.5) (width 0.2) (layer "F.Cu") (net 16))
 (segment (start 121.5 77.5) (end 121.5 88.001) (width 0.2) (layer "F.Cu") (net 16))
 (via (at 132.5 66.5) (size 0.6) (drill 0.3) (layers "F.Cu" "B.Cu") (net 16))
 (segment (start 132.5 63.8) (end 132.5 66.5) (width 0.2) (layer "B.Cu") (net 16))
 (segment (start 128.9 103.6) (end 128.9 99.425) (width 0.2) (layer "B.Cu") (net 10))
 (segment (start 127.9 106.3) (end 127.9 104.6) (width 0.2) (layer "B.Cu") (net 10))
 (segment (start 127.9 104.6) (end 128.9 103.6) (width 0.2) (layer "B.Cu") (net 10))
 (segment (start 130.3 74.121) (end 132.937 71.484) (width 0.2) (layer "B.Cu") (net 31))
 (segment (start 128.9 97.6) (end 130.3 96.2) (width 0.2) (layer "B.Cu") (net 31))
 (segment (start 130.3 96.2) (end 130.3 74.121) (width 0.2) (layer "B.Cu") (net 31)))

